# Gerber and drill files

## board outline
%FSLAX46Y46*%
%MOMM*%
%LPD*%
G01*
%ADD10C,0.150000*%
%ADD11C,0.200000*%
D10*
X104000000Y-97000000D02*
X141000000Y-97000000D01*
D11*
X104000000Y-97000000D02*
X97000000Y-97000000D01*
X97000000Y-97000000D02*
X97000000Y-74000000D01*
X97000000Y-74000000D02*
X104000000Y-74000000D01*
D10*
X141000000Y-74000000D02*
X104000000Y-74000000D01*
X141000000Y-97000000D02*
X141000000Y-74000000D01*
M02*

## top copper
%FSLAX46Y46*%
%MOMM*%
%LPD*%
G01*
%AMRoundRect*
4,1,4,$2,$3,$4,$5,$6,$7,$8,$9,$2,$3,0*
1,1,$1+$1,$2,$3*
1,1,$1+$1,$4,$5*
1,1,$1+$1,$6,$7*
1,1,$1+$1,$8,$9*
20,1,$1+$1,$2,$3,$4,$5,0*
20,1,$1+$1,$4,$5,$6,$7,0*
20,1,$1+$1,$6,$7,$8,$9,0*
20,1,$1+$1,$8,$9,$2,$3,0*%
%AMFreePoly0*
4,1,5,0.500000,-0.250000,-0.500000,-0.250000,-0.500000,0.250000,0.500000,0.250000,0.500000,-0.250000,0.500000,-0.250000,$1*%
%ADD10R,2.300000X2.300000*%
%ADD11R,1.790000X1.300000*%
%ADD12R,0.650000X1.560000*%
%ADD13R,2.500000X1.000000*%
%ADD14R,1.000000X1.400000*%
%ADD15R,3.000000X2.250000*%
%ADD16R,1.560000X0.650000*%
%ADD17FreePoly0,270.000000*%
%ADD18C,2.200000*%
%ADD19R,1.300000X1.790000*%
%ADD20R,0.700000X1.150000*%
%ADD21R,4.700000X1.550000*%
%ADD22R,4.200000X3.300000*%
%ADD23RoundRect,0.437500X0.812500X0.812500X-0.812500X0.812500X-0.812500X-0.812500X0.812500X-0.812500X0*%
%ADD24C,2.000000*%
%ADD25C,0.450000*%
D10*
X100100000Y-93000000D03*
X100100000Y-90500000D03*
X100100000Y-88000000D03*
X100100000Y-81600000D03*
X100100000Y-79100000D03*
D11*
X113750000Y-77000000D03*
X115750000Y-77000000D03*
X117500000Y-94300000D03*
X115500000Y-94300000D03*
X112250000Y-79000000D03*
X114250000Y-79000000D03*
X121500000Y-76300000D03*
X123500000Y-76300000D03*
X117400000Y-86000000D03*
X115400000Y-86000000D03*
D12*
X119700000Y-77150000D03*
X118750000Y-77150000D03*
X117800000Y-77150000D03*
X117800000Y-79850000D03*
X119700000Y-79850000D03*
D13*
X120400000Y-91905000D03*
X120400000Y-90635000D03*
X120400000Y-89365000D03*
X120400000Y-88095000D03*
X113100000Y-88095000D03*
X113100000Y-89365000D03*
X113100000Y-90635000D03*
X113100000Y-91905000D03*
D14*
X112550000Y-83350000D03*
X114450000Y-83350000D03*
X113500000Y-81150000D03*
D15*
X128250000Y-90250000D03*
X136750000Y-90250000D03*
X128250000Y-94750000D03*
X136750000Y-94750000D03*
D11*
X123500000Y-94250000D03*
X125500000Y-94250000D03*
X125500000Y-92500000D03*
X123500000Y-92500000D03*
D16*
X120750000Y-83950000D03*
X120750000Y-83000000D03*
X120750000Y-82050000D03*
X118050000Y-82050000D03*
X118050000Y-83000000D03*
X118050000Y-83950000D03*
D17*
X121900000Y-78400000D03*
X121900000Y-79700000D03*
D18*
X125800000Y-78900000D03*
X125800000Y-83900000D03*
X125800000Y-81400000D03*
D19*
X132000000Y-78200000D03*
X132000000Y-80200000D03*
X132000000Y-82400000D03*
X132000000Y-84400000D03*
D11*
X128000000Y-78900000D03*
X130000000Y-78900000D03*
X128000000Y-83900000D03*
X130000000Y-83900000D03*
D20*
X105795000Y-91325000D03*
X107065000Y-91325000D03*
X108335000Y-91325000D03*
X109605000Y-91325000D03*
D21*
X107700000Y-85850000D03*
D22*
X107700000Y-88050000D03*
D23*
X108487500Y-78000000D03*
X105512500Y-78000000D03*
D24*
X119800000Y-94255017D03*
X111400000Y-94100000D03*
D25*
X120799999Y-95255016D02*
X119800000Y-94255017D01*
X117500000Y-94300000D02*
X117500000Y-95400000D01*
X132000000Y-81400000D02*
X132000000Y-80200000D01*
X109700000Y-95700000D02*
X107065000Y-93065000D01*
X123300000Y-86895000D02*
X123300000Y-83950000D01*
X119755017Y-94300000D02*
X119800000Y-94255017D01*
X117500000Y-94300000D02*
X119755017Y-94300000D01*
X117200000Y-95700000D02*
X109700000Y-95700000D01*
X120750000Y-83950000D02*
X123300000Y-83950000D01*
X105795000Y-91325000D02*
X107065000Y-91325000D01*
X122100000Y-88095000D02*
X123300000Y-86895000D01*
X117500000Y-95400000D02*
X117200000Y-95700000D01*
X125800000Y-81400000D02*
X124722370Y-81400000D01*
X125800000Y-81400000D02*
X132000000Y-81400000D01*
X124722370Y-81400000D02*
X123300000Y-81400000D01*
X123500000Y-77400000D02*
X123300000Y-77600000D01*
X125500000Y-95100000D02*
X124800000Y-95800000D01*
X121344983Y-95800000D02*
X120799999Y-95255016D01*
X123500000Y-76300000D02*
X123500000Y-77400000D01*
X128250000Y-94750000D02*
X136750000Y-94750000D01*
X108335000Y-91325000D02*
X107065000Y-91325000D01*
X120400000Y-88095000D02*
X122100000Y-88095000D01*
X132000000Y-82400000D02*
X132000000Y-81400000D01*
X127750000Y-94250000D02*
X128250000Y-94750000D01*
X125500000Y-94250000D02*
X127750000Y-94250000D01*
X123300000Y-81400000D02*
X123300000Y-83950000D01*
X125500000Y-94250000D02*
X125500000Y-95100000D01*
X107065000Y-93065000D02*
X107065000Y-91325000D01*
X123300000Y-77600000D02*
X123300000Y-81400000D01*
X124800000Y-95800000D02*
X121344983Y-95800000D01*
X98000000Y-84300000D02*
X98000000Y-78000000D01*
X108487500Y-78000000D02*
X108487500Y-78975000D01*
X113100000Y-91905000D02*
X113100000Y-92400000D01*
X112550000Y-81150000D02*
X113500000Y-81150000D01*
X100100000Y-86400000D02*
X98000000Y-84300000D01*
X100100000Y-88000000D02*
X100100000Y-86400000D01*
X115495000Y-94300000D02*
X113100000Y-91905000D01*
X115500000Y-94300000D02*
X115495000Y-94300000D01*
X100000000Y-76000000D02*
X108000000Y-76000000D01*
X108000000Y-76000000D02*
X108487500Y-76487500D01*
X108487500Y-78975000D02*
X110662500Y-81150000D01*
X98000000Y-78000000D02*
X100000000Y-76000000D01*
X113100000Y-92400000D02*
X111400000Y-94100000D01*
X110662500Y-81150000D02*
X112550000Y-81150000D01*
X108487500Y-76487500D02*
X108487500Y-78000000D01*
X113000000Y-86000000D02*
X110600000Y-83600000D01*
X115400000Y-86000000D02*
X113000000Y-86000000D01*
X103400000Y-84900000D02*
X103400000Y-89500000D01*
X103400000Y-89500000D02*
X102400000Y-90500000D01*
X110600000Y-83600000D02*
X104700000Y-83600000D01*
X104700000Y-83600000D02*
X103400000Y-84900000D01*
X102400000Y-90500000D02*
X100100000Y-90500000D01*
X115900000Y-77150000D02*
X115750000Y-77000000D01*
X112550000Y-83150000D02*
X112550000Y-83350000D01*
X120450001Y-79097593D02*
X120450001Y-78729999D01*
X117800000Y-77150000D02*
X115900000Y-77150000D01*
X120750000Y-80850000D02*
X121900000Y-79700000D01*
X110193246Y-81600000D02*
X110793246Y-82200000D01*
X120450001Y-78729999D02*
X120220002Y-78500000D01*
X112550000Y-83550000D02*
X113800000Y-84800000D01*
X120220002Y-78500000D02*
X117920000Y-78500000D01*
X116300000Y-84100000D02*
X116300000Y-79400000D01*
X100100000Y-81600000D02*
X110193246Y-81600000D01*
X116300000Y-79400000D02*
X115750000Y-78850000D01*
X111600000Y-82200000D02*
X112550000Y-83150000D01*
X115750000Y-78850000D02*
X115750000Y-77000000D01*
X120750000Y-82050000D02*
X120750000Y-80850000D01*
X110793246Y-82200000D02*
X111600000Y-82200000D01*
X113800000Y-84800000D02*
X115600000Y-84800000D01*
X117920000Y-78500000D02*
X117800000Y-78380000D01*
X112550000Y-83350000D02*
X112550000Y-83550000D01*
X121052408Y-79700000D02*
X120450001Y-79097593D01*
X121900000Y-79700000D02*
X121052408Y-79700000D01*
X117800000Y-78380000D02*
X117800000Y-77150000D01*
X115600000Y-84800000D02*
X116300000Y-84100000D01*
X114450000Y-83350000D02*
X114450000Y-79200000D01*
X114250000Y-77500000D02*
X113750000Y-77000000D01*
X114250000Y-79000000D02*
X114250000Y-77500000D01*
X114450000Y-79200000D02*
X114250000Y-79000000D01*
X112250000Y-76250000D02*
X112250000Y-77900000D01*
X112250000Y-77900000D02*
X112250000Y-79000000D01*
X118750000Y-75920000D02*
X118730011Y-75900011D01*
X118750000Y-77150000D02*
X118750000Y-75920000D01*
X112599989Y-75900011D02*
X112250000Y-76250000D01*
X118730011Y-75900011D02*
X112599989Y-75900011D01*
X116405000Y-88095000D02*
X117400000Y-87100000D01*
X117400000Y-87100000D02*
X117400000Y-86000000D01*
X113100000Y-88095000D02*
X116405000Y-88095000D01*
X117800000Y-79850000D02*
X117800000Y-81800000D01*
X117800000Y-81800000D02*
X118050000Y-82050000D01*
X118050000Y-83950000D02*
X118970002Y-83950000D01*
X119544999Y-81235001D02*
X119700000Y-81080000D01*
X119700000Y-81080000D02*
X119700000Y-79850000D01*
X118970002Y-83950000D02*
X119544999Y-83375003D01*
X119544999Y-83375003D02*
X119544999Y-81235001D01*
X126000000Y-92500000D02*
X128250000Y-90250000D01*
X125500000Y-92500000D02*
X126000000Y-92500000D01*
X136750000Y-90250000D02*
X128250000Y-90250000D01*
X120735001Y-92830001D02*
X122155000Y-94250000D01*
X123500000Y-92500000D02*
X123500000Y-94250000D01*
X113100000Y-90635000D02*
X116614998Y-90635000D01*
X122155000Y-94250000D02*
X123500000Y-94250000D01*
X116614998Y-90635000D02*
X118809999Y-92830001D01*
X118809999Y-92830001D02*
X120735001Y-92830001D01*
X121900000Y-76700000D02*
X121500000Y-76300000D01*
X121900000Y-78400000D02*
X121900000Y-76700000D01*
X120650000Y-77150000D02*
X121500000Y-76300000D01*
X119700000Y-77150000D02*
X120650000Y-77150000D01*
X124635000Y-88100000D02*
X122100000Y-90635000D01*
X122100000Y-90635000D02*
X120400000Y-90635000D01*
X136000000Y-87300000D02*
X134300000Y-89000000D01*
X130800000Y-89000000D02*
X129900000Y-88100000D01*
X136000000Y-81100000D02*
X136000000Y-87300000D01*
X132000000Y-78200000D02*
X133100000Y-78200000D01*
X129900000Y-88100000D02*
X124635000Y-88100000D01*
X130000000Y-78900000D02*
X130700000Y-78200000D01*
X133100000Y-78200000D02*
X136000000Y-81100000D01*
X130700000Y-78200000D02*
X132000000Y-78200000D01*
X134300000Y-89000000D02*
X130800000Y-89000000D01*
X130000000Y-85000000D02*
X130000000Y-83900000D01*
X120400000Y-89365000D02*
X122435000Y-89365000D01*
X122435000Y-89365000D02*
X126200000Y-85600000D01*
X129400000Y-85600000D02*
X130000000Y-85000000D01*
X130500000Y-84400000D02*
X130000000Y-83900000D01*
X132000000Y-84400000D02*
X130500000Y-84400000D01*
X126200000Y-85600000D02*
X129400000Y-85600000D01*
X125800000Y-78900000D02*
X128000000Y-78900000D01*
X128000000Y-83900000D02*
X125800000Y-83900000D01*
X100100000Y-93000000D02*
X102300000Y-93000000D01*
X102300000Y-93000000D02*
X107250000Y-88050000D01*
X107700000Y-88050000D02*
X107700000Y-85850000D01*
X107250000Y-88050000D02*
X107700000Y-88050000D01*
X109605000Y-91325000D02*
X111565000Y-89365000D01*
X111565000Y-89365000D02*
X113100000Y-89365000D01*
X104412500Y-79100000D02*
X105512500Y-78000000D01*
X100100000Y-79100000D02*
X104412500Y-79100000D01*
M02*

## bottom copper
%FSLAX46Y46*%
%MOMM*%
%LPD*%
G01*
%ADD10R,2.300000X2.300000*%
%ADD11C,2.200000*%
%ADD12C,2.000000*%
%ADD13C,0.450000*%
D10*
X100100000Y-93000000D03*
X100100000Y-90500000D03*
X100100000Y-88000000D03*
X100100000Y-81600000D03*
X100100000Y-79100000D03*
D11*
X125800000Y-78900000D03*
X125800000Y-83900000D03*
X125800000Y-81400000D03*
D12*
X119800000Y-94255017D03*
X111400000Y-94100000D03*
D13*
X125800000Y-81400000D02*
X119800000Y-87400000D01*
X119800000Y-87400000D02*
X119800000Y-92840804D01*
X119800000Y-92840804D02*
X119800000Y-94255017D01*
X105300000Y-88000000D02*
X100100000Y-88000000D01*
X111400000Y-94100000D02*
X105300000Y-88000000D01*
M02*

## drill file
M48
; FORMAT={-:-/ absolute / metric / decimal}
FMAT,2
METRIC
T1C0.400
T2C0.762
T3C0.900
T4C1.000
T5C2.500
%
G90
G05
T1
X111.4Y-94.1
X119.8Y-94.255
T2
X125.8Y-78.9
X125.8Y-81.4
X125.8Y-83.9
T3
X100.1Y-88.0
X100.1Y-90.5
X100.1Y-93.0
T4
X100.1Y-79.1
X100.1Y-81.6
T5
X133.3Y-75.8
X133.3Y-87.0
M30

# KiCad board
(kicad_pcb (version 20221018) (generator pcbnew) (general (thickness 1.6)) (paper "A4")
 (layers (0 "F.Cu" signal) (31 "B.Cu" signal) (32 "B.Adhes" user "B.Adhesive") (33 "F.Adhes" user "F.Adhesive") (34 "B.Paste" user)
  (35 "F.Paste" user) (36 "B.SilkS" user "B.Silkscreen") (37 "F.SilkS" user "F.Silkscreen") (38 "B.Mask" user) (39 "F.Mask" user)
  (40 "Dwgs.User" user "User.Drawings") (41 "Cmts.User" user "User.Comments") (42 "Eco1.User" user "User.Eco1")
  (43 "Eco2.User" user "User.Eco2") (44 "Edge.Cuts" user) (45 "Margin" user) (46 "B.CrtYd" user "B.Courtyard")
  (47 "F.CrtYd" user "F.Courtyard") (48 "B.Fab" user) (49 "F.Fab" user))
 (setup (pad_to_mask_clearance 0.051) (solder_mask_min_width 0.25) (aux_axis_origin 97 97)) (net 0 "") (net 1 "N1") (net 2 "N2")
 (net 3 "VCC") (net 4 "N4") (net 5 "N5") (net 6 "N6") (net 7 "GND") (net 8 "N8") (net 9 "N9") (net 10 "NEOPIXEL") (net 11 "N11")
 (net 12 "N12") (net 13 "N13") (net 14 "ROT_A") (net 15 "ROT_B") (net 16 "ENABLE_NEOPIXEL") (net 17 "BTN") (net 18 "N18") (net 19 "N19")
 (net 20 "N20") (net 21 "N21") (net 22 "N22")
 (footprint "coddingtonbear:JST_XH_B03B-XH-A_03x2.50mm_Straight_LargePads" (layer "F.Cu") (at 100.1 93 90)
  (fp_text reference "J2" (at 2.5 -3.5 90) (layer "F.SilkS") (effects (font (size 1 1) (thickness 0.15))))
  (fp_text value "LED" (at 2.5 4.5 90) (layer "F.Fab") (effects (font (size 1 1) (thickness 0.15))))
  (pad "1" thru_hole rect (at 0 0 90) (size 2.3 2.3) (drill 0.9) (layers "*.Cu" "*.Mask") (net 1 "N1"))
  (pad "2" thru_hole rect (at 2.5 0 90) (size 2.3 2.3) (drill 0.9) (layers "*.Cu" "*.Mask") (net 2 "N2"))
  (pad "3" thru_hole rect (at 5 0 90) (size 2.3 2.3) (drill 0.9) (layers "*.Cu" "*.Mask") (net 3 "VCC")))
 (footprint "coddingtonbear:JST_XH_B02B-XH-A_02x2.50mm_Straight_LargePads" (layer "F.Cu") (at 100.1 81.6 90)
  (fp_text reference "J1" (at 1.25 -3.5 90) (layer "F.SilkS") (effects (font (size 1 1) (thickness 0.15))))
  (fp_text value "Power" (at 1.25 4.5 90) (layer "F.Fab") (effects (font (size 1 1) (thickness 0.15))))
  (pad "1" thru_hole rect (at 0 0 90) (size 2.3 2.3) (drill 1) (layers "*.Cu" "*.Mask") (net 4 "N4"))
  (pad "2" thru_hole rect (at 2.5 0 90) (size 2.3 2.3) (drill 1) (layers "*.Cu" "*.Mask") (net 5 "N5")))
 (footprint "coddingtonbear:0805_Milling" (layer "F.Cu") (at 114.75 77)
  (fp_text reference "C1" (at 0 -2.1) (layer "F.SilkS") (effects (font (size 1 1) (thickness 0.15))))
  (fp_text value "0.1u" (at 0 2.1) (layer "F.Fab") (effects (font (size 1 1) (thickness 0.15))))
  (pad "1" smd rect (at -1 0) (size 1.79 1.3) (layers "F.Cu" "F.Paste" "F.Mask") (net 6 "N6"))
  (pad "2" smd rect (at 1 0) (size 1.79 1.3) (layers "F.Cu" "F.Paste" "F.Mask") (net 4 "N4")))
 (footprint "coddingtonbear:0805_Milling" (layer "F.Cu") (at 116.5 94.3 180)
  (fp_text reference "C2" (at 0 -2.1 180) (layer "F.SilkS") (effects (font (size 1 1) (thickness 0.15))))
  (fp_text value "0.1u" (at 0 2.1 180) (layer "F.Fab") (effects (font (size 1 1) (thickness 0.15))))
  (pad "1" smd rect (at -1 0 180) (size 1.79 1.3) (layers "F.Cu" "F.Paste" "F.Mask") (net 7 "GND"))
  (pad "2" smd rect (at 1 0 180) (size 1.79 1.3) (layers "F.Cu" "F.Paste" "F.Mask") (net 3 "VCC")))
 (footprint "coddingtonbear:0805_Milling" (layer "F.Cu") (at 113.25 79)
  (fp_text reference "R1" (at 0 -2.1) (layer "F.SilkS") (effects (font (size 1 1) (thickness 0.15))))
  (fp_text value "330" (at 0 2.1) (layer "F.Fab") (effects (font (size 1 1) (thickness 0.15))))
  (pad "1" smd rect (at -1 0) (size 1.79 1.3) (layers "F.Cu" "F.Paste" "F.Mask") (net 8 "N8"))
  (pad "2" smd rect (at 1 0) (size 1.79 1.3) (layers "F.Cu" "F.Paste" "F.Mask") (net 6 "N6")))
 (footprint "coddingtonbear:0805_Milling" (layer "F.Cu") (at 122.5 76.3)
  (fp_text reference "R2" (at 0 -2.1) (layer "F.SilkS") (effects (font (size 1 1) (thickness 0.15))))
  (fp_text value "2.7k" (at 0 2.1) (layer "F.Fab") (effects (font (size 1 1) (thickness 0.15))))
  (pad "1" smd rect (at -1 0) (size 1.79 1.3) (layers "F.Cu" "F.Paste" "F.Mask") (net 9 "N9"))
  (pad "2" smd rect (at 1 0) (size 1.79 1.3) (layers "F.Cu" "F.Paste" "F.Mask") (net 7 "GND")))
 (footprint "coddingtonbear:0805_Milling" (layer "F.Cu") (at 116.4 86 180)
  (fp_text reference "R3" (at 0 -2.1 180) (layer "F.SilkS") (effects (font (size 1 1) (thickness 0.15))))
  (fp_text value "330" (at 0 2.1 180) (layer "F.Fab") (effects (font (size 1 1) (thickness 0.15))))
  (pad "1" smd rect (at -1 0 180) (size 1.79 1.3) (layers "F.Cu" "F.Paste" "F.Mask") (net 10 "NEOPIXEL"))
  (pad "2" smd rect (at 1 0 180) (size 1.79 1.3) (layers "F.Cu" "F.Paste" "F.Mask") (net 2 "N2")))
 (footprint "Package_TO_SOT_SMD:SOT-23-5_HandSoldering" (layer "F.Cu") (at 118.75 78.5 -90)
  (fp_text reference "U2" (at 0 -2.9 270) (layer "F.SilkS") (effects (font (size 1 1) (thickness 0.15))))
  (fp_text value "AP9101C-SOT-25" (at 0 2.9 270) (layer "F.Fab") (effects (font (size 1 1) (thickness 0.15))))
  (pad "1" smd rect (at -1.35 -0.95 270) (size 1.56 0.65) (layers "F.Cu" "F.Paste" "F.Mask") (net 9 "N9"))
  (pad "2" smd rect (at -1.35 0 270) (size 1.56 0.65) (layers "F.Cu" "F.Paste" "F.Mask") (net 8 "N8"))
  (pad "3" smd rect (at -1.35 0.95 270) (size 1.56 0.65) (layers "F.Cu" "F.Paste" "F.Mask") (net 4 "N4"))
  (pad "4" smd rect (at 1.35 0.95 270) (size 1.56 0.65) (layers "F.Cu" "F.Paste" "F.Mask") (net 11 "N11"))
  (pad "5" smd rect (at 1.35 -0.95 270) (size 1.56 0.65) (layers "F.Cu" "F.Paste" "F.Mask") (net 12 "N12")))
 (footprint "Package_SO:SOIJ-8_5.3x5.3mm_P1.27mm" (layer "F.Cu") (at 116.75 90 180)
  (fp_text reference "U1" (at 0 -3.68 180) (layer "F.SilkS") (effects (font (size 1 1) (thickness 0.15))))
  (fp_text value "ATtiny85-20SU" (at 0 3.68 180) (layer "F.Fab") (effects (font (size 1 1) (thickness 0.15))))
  (pad "1" smd rect (at -3.65 -1.905 180) (size 2.5 1) (layers "F.Cu" "F.Paste" "F.Mask") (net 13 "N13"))
  (pad "2" smd rect (at -3.65 -0.635 180) (size 2.5 1) (layers "F.Cu" "F.Paste" "F.Mask") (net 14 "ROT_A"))
  (pad "3" smd rect (at -3.65 0.635 180) (size 2.5 1) (layers "F.Cu" "F.Paste" "F.Mask") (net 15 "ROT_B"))
  (pad "4" smd rect (at -3.65 1.905 180) (size 2.5 1) (layers "F.Cu" "F.Paste" "F.Mask") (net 7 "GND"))
  (pad "5" smd rect (at 3.65 1.905 180) (size 2.5 1) (layers "F.Cu" "F.Paste" "F.Mask") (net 10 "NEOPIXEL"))
  (pad "6" smd rect (at 3.65 0.635 180) (size 2.5 1) (layers "F.Cu" "F.Paste" "F.Mask") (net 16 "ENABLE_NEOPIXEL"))
  (pad "7" smd rect (at 3.65 -0.635 180) (size 2.5 1) (layers "F.Cu" "F.Paste" "F.Mask") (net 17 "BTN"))
  (pad "8" smd rect (at 3.65 -1.905 180) (size 2.5 1) (layers "F.Cu" "F.Paste" "F.Mask") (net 3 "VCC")))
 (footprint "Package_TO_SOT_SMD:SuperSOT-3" (layer "F.Cu") (at 113.5 82.25 90)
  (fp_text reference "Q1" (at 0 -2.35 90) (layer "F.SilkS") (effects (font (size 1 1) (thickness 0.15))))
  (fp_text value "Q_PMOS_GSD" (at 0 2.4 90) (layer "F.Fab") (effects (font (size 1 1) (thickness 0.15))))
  (pad "1" smd rect (at -1.1 -0.95 90) (size 1.4 1) (layers "F.Cu" "F.Paste" "F.Mask") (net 4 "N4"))
  (pad "2" smd rect (at -1.1 0.95 90) (size 1.4 1) (layers "F.Cu" "F.Paste" "F.Mask") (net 6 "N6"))
  (pad "3" smd rect (at 1.1 0 90) (size 1.4 1) (layers "F.Cu" "F.Paste" "F.Mask") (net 3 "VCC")))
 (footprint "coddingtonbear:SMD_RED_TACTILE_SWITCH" (layer "F.Cu") (at 132.5 92.5)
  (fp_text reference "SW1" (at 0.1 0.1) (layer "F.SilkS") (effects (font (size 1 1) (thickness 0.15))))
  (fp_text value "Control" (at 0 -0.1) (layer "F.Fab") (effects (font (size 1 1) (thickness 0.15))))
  (pad "1" smd rect (at -4.25 -2.25) (size 3 2.25) (layers "F.Cu" "F.Paste" "F.Mask") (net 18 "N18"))
  (pad "1" smd rect (at 4.25 -2.25) (size 3 2.25) (layers "F.Cu" "F.Paste" "F.Mask") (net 18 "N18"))
  (pad "2" smd rect (at -4.25 2.25) (size 3 2.25) (layers "F.Cu" "F.Paste" "F.Mask") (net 7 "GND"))
  (pad "2" smd rect (at 4.25 2.25) (size 3 2.25) (layers "F.Cu" "F.Paste" "F.Mask") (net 7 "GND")))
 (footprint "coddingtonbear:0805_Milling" (layer "F.Cu") (at 124.5 94.25)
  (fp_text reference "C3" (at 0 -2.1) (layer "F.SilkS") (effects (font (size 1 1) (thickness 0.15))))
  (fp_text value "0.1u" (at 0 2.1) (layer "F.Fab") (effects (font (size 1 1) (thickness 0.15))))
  (pad "1" smd rect (at -1 0) (size 1.79 1.3) (layers "F.Cu" "F.Paste" "F.Mask") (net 17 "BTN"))
  (pad "2" smd rect (at 1 0) (size 1.79 1.3) (layers "F.Cu" "F.Paste" "F.Mask") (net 7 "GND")))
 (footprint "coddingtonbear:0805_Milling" (layer "F.Cu") (at 124.5 92.5 180)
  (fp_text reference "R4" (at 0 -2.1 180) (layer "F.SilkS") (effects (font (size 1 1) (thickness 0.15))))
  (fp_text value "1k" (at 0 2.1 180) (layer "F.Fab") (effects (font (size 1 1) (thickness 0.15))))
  (pad "1" smd rect (at -1 0 180) (size 1.79 1.3) (layers "F.Cu" "F.Paste" "F.Mask") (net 18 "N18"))
  (pad "2" smd rect (at 1 0 180) (size 1.79 1.3) (layers "F.Cu" "F.Paste" "F.Mask") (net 17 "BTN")))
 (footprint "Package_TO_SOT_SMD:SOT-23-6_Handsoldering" (layer "F.Cu") (at 119.4 83 180)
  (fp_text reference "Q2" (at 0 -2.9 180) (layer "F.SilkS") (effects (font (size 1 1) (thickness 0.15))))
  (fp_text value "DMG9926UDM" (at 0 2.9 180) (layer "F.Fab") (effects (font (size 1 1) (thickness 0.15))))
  (pad "1" smd rect (at -1.35 -0.95 180) (size 1.56 0.65) (layers "F.Cu" "F.Paste" "F.Mask") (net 7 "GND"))
  (pad "2" smd rect (at -1.35 0 180) (size 1.56 0.65) (layers "F.Cu" "F.Paste" "F.Mask") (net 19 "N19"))
  (pad "3" smd rect (at -1.35 0.95 180) (size 1.56 0.65) (layers "F.Cu" "F.Paste" "F.Mask") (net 4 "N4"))
  (pad "4" smd rect (at 1.35 0.95 180) (size 1.56 0.65) (layers "F.Cu" "F.Paste" "F.Mask") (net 11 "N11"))
  (pad "5" smd rect (at 1.35 0 180) (size 1.56 0.65) (layers "F.Cu" "F.Paste" "F.Mask") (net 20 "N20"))
  (pad "6" smd rect (at 1.35 -0.95 180) (size 1.56 0.65) (layers "F.Cu" "F.Paste" "F.Mask") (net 12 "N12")))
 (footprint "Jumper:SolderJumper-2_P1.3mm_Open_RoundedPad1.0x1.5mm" (layer "F.Cu") (at 121.9 79.05 -90)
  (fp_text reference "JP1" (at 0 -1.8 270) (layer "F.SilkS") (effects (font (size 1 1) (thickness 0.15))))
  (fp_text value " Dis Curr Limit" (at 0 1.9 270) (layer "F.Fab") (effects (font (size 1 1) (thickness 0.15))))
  (pad "1" smd custom (at -0.65 0 270) (size 1 0.5) (layers "F.Cu" "F.Mask") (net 9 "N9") (zone_connect 0) (thermal_bridge_angle 45)
   (options (clearance outline) (anchor rect)) (primitives))
  (pad "2" smd custom (at 0.65 0 270) (size 1 0.5) (layers "F.Cu" "F.Mask") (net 4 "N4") (zone_connect 0) (thermal_bridge_angle 45)
   (options (clearance outline) (anchor rect)) (primitives)))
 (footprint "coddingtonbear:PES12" (layer "F.Cu") (at 133.3 81.4 -90)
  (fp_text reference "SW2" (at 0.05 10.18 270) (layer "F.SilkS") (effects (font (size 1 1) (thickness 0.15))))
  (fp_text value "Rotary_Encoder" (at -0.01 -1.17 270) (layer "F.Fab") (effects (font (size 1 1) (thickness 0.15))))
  (pad "" np_thru_hole circle (at -5.6 0 270) (size 2.5 2.5) (drill 2.5) (layers "*.Cu" "*.Mask"))
  (pad "" np_thru_hole circle (at 5.6 0 270) (size 2.5 2.5) (drill 2.5) (layers "*.Cu" "*.Mask"))
  (pad "A" thru_hole circle (at -2.5 7.5 270) (size 2.2 2.2) (drill 0.762) (layers "*.Cu" "*.Mask") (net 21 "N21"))
  (pad "B" thru_hole circle (at 2.5 7.5 270) (size 2.2 2.2) (drill 0.762) (layers "*.Cu" "*.Mask") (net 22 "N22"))
  (pad "C" thru_hole circle (at 0 7.5 270) (size 2.2 2.2) (drill 0.762) (layers "*.Cu" "*.Mask") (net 7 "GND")))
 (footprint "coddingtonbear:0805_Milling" (layer "F.Cu") (at 132 79.2 -90)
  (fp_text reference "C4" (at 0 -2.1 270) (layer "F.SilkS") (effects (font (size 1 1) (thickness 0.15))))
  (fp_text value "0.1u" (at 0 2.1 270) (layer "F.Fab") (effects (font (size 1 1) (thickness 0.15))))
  (pad "1" smd rect (at -1 0 270) (size 1.79 1.3) (layers "F.Cu" "F.Paste" "F.Mask") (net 14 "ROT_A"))
  (pad "2" smd rect (at 1 0 270) (size 1.79 1.3) (layers "F.Cu" "F.Paste" "F.Mask") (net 7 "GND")))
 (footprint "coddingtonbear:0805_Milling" (layer "F.Cu") (at 132 83.4 -90)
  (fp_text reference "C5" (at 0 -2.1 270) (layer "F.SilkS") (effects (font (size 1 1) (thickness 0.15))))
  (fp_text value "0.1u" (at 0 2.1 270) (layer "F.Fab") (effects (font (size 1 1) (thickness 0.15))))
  (pad "1" smd rect (at -1 0 270) (size 1.79 1.3) (layers "F.Cu" "F.Paste" "F.Mask") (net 7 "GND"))
  (pad "2" smd rect (at 1 0 270) (size 1.79 1.3) (layers "F.Cu" "F.Paste" "F.Mask") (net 15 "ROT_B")))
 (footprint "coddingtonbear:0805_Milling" (layer "F.Cu") (at 129 78.9)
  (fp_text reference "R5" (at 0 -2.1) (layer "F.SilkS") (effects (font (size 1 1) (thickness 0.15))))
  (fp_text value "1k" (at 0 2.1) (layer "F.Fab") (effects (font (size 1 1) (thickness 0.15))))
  (pad "1" smd rect (at -1 0) (size 1.79 1.3) (layers "F.Cu" "F.Paste" "F.Mask") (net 21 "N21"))
  (pad "2" smd rect (at 1 0) (size 1.79 1.3) (layers "F.Cu" "F.Paste" "F.Mask") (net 14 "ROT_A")))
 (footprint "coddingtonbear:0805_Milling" (layer "F.Cu") (at 129 83.9)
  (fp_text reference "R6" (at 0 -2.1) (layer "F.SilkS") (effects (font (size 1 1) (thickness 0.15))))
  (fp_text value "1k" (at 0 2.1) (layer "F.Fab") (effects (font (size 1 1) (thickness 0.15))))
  (pad "1" smd rect (at -1 0) (size 1.79 1.3) (layers "F.Cu" "F.Paste" "F.Mask") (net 22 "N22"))
  (pad "2" smd rect (at 1 0) (size 1.79 1.3) (layers "F.Cu" "F.Paste" "F.Mask") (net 15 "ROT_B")))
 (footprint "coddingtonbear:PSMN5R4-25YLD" (layer "F.Cu") (at 107.7 88.5)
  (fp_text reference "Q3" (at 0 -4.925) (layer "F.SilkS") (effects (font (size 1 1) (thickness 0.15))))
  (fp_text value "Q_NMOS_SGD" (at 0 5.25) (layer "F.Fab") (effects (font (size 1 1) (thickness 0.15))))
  (pad "" smd rect (at -1.875 -2.9) (size 0.6 0.9) (layers "F.Paste"))
  (pad "" smd rect (at -1.15 -1.05 90) (size 0.6 0.9) (layers "F.Paste"))
  (pad "" smd rect (at -1.15 -0.2 90) (size 0.6 0.9) (layers "F.Paste"))
  (pad "" smd rect (at -1.15 0.65 90) (size 0.6 0.9) (layers "F.Paste"))
  (pad "" smd rect (at -0.6 -2.9) (size 0.6 0.9) (layers "F.Paste"))
  (pad "" smd rect (at 0 -1.05 90) (size 0.6 0.9) (layers "F.Paste"))
  (pad "" smd rect (at 0 -0.2 90) (size 0.6 0.9) (layers "F.Paste"))
  (pad "" smd rect (at 0 0.65 90) (size 0.6 0.9) (layers "F.Paste"))
  (pad "" smd rect (at 0.6 -2.9) (size 0.6 0.9) (layers "F.Paste"))
  (pad "" smd rect (at 1.15 -1.05 90) (size 0.6 0.9) (layers "F.Paste"))
  (pad "" smd rect (at 1.15 -0.2 90) (size 0.6 0.9) (layers "F.Paste"))
  (pad "" smd rect (at 1.15 0.65 90) (size 0.6 0.9) (layers "F.Paste"))
  (pad "" smd rect (at 1.875 -2.9) (size 0.6 0.9) (layers "F.Paste"))
  (pad "1" smd rect (at -1.905 2.825) (size 0.7 1.15) (layers "F.Cu" "F.Paste" "F.Mask") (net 7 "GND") (solder_mask_margin 0.075)
   (solder_paste_margin -0.05))
  (pad "1" smd rect (at -0.635 2.825) (size 0.7 1.15) (layers "F.Cu" "F.Paste" "F.Mask") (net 7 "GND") (solder_mask_margin 0.075)
   (solder_paste_margin -0.05))
  (pad "1" smd rect (at 0.635 2.825) (size 0.7 1.15) (layers "F.Cu" "F.Paste" "F.Mask") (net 7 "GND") (solder_mask_margin 0.075)
   (solder_paste_margin -0.05))
  (pad "2" smd rect (at 1.905 2.825) (size 0.7 1.15) (layers "F.Cu" "F.Paste" "F.Mask") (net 16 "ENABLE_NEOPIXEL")
   (solder_mask_margin 0.075) (solder_paste_margin -0.05))
  (pad "3" smd rect (at 0 -2.65) (size 4.7 1.55) (layers "F.Cu" "F.Mask") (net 1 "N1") (solder_mask_margin 0.075))
  (pad "3" smd rect (at 0 -0.45) (size 4.2 3.3) (layers "F.Cu" "F.Mask") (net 1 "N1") (solder_mask_margin 0.075)))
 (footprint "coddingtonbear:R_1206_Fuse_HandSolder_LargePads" (layer "F.Cu") (at 107 78 180)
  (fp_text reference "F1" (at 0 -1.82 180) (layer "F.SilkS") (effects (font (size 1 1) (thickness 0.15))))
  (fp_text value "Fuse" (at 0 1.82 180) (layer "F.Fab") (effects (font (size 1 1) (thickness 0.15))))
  (pad "1" smd roundrect (at -1.4875 0 180) (size 2.5 2.5) (layers "F.Cu" "F.Paste" "F.Mask") (roundrect_rratio 0.175) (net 3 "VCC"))
  (pad "2" smd roundrect (at 1.4875 0 180) (size 2.5 2.5) (layers "F.Cu" "F.Paste" "F.Mask") (roundrect_rratio 0.175) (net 5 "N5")))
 (gr_line (start 104 97) (end 141 97) (stroke (width 0.15) (type solid)) (layer "Edge.Cuts"))
 (gr_line (start 104 97) (end 97 97) (stroke (width 0.2) (type solid)) (layer "Edge.Cuts"))
 (gr_line (start 97 97) (end 97 74) (stroke (width 0.2) (type solid)) (layer "Edge.Cuts"))
 (gr_line (start 97 74) (end 104 74) (stroke (width 0.2) (type solid)) (layer "Edge.Cuts"))
 (gr_line (start 141 74) (end 104 74) (stroke (width 0.15) (type solid)) (layer "Edge.Cuts"))
 (gr_line (start 141 97) (end 141 74) (stroke (width 0.15) (type solid)) (layer "Edge.Cuts"))
 (segment (start 120.799999 95.255016) (end 119.8 94.255017) (width 0.45) (layer "F.Cu") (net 7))
 (segment (start 117.5 94.3) (end 117.5 95.4) (width 0.45) (layer "F.Cu") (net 7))
 (segment (start 132 81.4) (end 132 80.2) (width 0.45) (layer "F.Cu") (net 7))
 (segment (start 109.7 95.7) (end 107.065 93.065) (width 0.45) (layer "F.Cu") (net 7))
 (segment (start 123.3 86.895) (end 123.3 83.95) (width 0.45) (layer "F.Cu") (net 7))
 (segment (start 119.755017 94.3) (end 119.8 94.255017) (width 0.45) (layer "F.Cu") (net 7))
 (segment (start 117.5 94.3) (end 119.755017 94.3) (width 0.45) (layer "F.Cu") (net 7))
 (segment (start 117.2 95.7) (end 109.7 95.7) (width 0.45) (layer "F.Cu") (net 7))
 (segment (start 120.75 83.95) (end 123.3 83.95) (width 0.45) (layer "F.Cu") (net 7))
 (segment (start 105.795 91.325) (end 107.065 91.325) (width 0.45) (layer "F.Cu") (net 7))
 (segment (start 122.1 88.095) (end 123.3 86.895) (width 0.45) (layer "F.Cu") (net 7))
 (segment (start 117.5 95.4) (end 117.2 95.7) (width 0.45) (layer "F.Cu") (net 7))
 (segment (start 125.8 81.4) (end 124.72237 81.4) (width 0.45) (layer "F.Cu") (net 7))
 (segment (start 125.8 81.4) (end 132 81.4) (width 0.45) (layer "F.Cu") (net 7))
 (segment (start 124.72237 81.4) (end 123.3 81.4) (width 0.45) (layer "F.Cu") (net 7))
 (segment (start 123.5 77.4) (end 123.3 77.6) (width 0.45) (layer "F.Cu") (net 7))
 (segment (start 125.5 95.1) (end 124.8 95.8) (width 0.45) (layer "F.Cu") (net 7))
 (segment (start 121.344983 95.8) (end 120.799999 95.255016) (width 0.45) (layer "F.Cu") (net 7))
 (segment (start 123.5 76.3) (end 123.5 77.4) (width 0.45) (layer "F.Cu") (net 7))
 (segment (start 128.25 94.75) (end 136.75 94.75) (width 0.45) (layer "F.Cu") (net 7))
 (segment (start 108.335 91.325) (end 107.065 91.325) (width 0.45) (layer "F.Cu") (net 7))
 (segment (start 120.4 88.095) (end 122.1 88.095) (width 0.45) (layer "F.Cu") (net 7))
 (segment (start 132 82.4) (end 132 81.4) (width 0.45) (layer "F.Cu") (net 7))
 (segment (start 127.75 94.25) (end 128.25 94.75) (width 0.45) (layer "F.Cu") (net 7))
 (segment (start 125.5 94.25) (end 127.75 94.25) (width 0.45) (layer "F.Cu") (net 7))
 (segment (start 123.3 81.4) (end 123.3 83.95) (width 0.45) (layer "F.Cu") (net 7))
 (segment (start 125.5 94.25) (end 125.5 95.1) (width 0.45) (layer "F.Cu") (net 7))
 (segment (start 107.065 93.065) (end 107.065 91.325) (width 0.45) (layer "F.Cu") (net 7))
 (segment (start 123.3 77.6) (end 123.3 81.4) (width 0.45) (layer "F.Cu") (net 7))
 (segment (start 124.8 95.8) (end 121.344983 95.8) (width 0.45) (layer "F.Cu") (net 7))
 (via (at 119.8 94.255017) (size 2) (drill 0.4) (layers "F.Cu" "B.Cu") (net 7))
 (segment (start 125.8 81.4) (end 119.8 87.4) (width 0.45) (layer "B.Cu") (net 7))
 (segment (start 119.8 87.4) (end 119.8 92.840804) (width 0.45) (layer "B.Cu") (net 7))
 (segment (start 119.8 92.840804) (end 119.8 94.255017) (width 0.45) (layer "B.Cu") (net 7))
 (segment (start 98 84.3) (end 98 78) (width 0.45) (layer "F.Cu") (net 3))
 (segment (start 108.4875 78) (end 108.4875 78.975) (width 0.45) (layer "F.Cu") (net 3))
 (segment (start 113.1 91.905) (end 113.1 92.4) (width 0.45) (layer "F.Cu") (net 3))
 (segment (start 112.55 81.15) (end 113.5 81.15) (width 0.45) (layer "F.Cu") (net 3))
 (segment (start 100.1 86.4) (end 98 84.3) (width 0.45) (layer "F.Cu") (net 3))
 (segment (start 100.1 88) (end 100.1 86.4) (width 0.45) (layer "F.Cu") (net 3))
 (segment (start 115.495 94.3) (end 113.1 91.905) (width 0.45) (layer "F.Cu") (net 3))
 (segment (start 115.5 94.3) (end 115.495 94.3) (width 0.45) (layer "F.Cu") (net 3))
 (segment (start 100 76) (end 108 76) (width 0.45) (layer "F.Cu") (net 3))
 (segment (start 108 76) (end 108.4875 76.4875) (width 0.45) (layer "F.Cu") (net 3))
 (segment (start 108.4875 78.975) (end 110.6625 81.15) (width 0.45) (layer "F.Cu") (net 3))
 (segment (start 98 78) (end 100 76) (width 0.45) (layer "F.Cu") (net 3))
 (segment (start 113.1 92.4) (end 111.4 94.1) (width 0.45) (layer "F.Cu") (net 3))
 (segment (start 110.6625 81.15) (end 112.55 81.15) (width 0.45) (layer "F.Cu") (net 3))
 (segment (start 108.4875 76.4875) (end 108.4875 78) (width 0.45) (layer "F.Cu") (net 3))
 (via (at 111.4 94.1) (size 2) (drill 0.4) (layers "F.Cu" "B.Cu") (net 3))
 (segment (start 105.3 88) (end 100.1 88) (width 0.45) (layer "B.Cu") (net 3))
 (segment (start 111.4 94.1) (end 105.3 88) (width 0.45) (layer "B.Cu") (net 3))
 (segment (start 113 86) (end 110.6 83.6) (width 0.45) (layer "F.Cu") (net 2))
 (segment (start 115.4 86) (end 113 86) (width 0.45) (layer "F.Cu") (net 2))
 (segment (start 103.4 84.9) (end 103.4 89.5) (width 0.45) (layer "F.Cu") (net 2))
 (segment (start 103.4 89.5) (end 102.4 90.5) (width 0.45) (layer "F.Cu") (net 2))
 (segment (start 110.6 83.6) (end 104.7 83.6) (width 0.45) (layer "F.Cu") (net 2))
 (segment (start 104.7 83.6) (end 103.4 84.9) (width 0.45) (layer "F.Cu") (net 2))
 (segment (start 102.4 90.5) (end 100.1 90.5) (width 0.45) (layer "F.Cu") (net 2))
 (segment (start 115.9 77.15) (end 115.75 77) (width 0.45) (layer "F.Cu") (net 4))
 (segment (start 112.55 83.15) (end 112.55 83.35) (width 0.45) (layer "F.Cu") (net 4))
 (segment (start 120.450001 79.097593) (end 120.450001 78.729999) (width 0.45) (layer "F.Cu") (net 4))
 (segment (start 117.8 77.15) (end 115.9 77.15) (width 0.45) (layer "F.Cu") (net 4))
 (segment (start 120.75 80.85) (end 121.9 79.7) (width 0.45) (layer "F.Cu") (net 4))
 (segment (start 110.193246 81.6) (end 110.793246 82.2) (width 0.45) (layer "F.Cu") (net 4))
 (segment (start 120.450001 78.729999) (end 120.220002 78.5) (width 0.45) (layer "F.Cu") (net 4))
 (segment (start 112.55 83.55) (end 113.8 84.8) (width 0.45) (layer "F.Cu") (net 4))
 (segment (start 120.220002 78.5) (end 117.92 78.5) (width 0.45) (layer "F.Cu") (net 4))
 (segment (start 116.3 84.1) (end 116.3 79.4) (width 0.45) (layer "F.Cu") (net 4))
 (segment (start 100.1 81.6) (end 110.193246 81.6) (width 0.45) (layer "F.Cu") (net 4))
 (segment (start 116.3 79.4) (end 115.75 78.85) (width 0.45) (layer "F.Cu") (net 4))
 (segment (start 111.6 82.2) (end 112.55 83.15) (width 0.45) (layer "F.Cu") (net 4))
 (segment (start 115.75 78.85) (end 115.75 77) (width 0.45) (layer "F.Cu") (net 4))
 (segment (start 120.75 82.05) (end 120.75 80.85) (width 0.45) (layer "F.Cu") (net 4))
 (segment (start 110.793246 82.2) (end 111.6 82.2) (width 0.45) (layer "F.Cu") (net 4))
 (segment (start 113.8 84.8) (end 115.6 84.8) (width 0.45) (layer "F.Cu") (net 4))
 (segment (start 117.92 78.5) (end 117.8 78.38) (width 0.45) (layer "F.Cu") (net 4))
 (segment (start 112.55 83.35) (end 112.55 83.55) (width 0.45) (layer "F.Cu") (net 4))
 (segment (start 121.052408 79.7) (end 120.450001 79.097593) (width 0.45) (layer "F.Cu") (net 4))
 (segment (start 121.9 79.7) (end 121.052408 79.7) (width 0.45) (layer "F.Cu") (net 4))
 (segment (start 117.8 78.38) (end 117.8 77.15) (width 0.45) (layer "F.Cu") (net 4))
 (segment (start 115.6 84.8) (end 116.3 84.1) (width 0.45) (layer "F.Cu") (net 4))
 (segment (start 114.45 83.35) (end 114.45 79.2) (width 0.45) (layer "F.Cu") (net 6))
 (segment (start 114.25 77.5) (end 113.75 77) (width 0.45) (layer "F.Cu") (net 6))
 (segment (start 114.25 79) (end 114.25 77.5) (width 0.45) (layer "F.Cu") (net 6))
 (segment (start 114.45 79.2) (end 114.25 79) (width 0.45) (layer "F.Cu") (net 6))
 (segment (start 112.25 76.25) (end 112.25 77.9) (width 0.45) (layer "F.Cu") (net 8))
 (segment (start 112.25 77.9) (end 112.25 79) (width 0.45) (layer "F.Cu") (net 8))
 (segment (start 118.75 75.92) (end 118.730011 75.900011) (width 0.45) (layer "F.Cu") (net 8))
 (segment (start 118.75 77.15) (end 118.75 75.92) (width 0.45) (layer "F.Cu") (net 8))
 (segment (start 112.599989 75.900011) (end 112.25 76.25) (width 0.45) (layer "F.Cu") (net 8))
 (segment (start 118.730011 75.900011) (end 112.599989 75.900011) (width 0.45) (layer "F.Cu") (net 8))
 (segment (start 116.405 88.095) (end 117.4 87.1) (width 0.45) (layer "F.Cu") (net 10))
 (segment (start 117.4 87.1) (end 117.4 86) (width 0.45) (layer "F.Cu") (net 10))
 (segment (start 113.1 88.095) (end 116.405 88.095) (width 0.45) (layer "F.Cu") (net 10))
 (segment (start 117.8 79.85) (end 117.8 81.8) (width 0.45) (layer "F.Cu") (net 11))
 (segment (start 117.8 81.8) (end 118.05 82.05) (width 0.45) (layer "F.Cu") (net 11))
 (segment (start 118.05 83.95) (end 118.970002 83.95) (width 0.45) (layer "F.Cu") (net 12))
 (segment (start 119.544999 81.235001) (end 119.7 81.08) (width 0.45) (layer "F.Cu") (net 12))
 (segment (start 119.7 81.08) (end 119.7 79.85) (width 0.45) (layer "F.Cu") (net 12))
 (segment (start 118.970002 83.95) (end 119.544999 83.375003) (width 0.45) (layer "F.Cu") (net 12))
 (segment (start 119.544999 83.375003) (end 119.544999 81.235001) (width 0.45) (layer "F.Cu") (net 12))
 (segment (start 126 92.5) (end 128.25 90.25) (width 0.45) (layer "F.Cu") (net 18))
 (segment (start 125.5 92.5) (end 126 92.5) (width 0.45) (layer "F.Cu") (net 18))
 (segment (start 136.75 90.25) (end 128.25 90.25) (width 0.45) (layer "F.Cu") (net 18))
 (segment (start 120.735001 92.830001) (end 122.155 94.25) (width 0.45) (layer "F.Cu") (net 17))
 (segment (start 123.5 92.5) (end 123.5 94.25) (width 0.45) (layer "F.Cu") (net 17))
 (segment (start 113.1 90.635) (end 116.614998 90.635) (width 0.45) (layer "F.Cu") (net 17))
 (segment (start 122.155 94.25) (end 123.5 94.25) (width 0.45) (layer "F.Cu") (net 17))
 (segment (start 116.614998 90.635) (end 118.809999 92.830001) (width 0.45) (layer "F.Cu") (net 17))
 (segment (start 118.809999 92.830001) (end 120.735001 92.830001) (width 0.45) (layer "F.Cu") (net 17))
 (segment (start 121.9 76.7) (end 121.5 76.3) (width 0.45) (layer "F.Cu") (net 9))
 (segment (start 121.9 78.4) (end 121.9 76.7) (width 0.45) (layer "F.Cu") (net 9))
 (segment (start 120.65 77.15) (end 121.5 76.3) (width 0.45) (layer "F.Cu") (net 9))
 (segment (start 119.7 77.15) (end 120.65 77.15) (width 0.45) (layer "F.Cu") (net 9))
 (segment (start 124.635 88.1) (end 122.1 90.635) (width 0.45) (layer "F.Cu") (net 14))
 (segment (start 122.1 90.635) (end 120.4 90.635) (width 0.45) (layer "F.Cu") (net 14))
 (segment (start 136 87.3) (end 134.3 89) (width 0.45) (layer "F.Cu") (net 14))
 (segment (start 130.8 89) (end 129.9 88.1) (width 0.45) (layer "F.Cu") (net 14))
 (segment (start 136 81.1) (end 136 87.3) (width 0.45) (layer "F.Cu") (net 14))
 (segment (start 132 78.2) (end 133.1 78.2) (width 0.45) (layer "F.Cu") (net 14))
 (segment (start 129.9 88.1) (end 124.635 88.1) (width 0.45) (layer "F.Cu") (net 14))
 (segment (start 130 78.9) (end 130.7 78.2) (width 0.45) (layer "F.Cu") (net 14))
 (segment (start 133.1 78.2) (end 136 81.1) (width 0.45) (layer "F.Cu") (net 14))
 (segment (start 130.7 78.2) (end 132 78.2) (width 0.45) (layer "F.Cu") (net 14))
 (segment (start 134.3 89) (end 130.8 89) (width 0.45) (layer "F.Cu") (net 14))
 (segment (start 130 85) (end 130 83.9) (width 0.45) (layer "F.Cu") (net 15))
 (segment (start 120.4 89.365) (end 122.435 89.365) (width 0.45) (layer "F.Cu") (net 15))
 (segment (start 122.435 89.365) (end 126.2 85.6) (width 0.45) (layer "F.Cu") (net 15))
 (segment (start 129.4 85.6) (end 130 85) (width 0.45) (layer "F.Cu") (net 15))
 (segment (start 130.5 84.4) (end 130 83.9) (width 0.45) (layer "F.Cu") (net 15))
 (segment (start 132 84.4) (end 130.5 84.4) (width 0.45) (layer "F.Cu") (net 15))
 (segment (start 126.2 85.6) (end 129.4 85.6) (width 0.45) (layer "F.Cu") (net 15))
 (segment (start 125.8 78.9) (end 128 78.9) (width 0.45) (layer "F.Cu") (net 21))
 (segment (start 128 83.9) (end 125.8 83.9) (width 0.45) (layer "F.Cu") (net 22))
 (segment (start 100.1 93) (end 102.3 93) (width 0.45) (layer "F.Cu") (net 1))
 (segment (start 102.3 93) (end 107.25 88.05) (width 0.45) (layer "F.Cu") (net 1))
 (segment (start 107.7 88.05) (end 107.7 85.85) (width 0.45) (layer "F.Cu") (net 1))
 (segment (start 107.25 88.05) (end 107.7 88.05) (width 0.45) (layer "F.Cu") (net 1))
 (segment (start 109.605 91.325) (end 111.565 89.365) (width 0.45) (layer "F.Cu") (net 16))
 (segment (start 111.565 89.365) (end 113.1 89.365) (width 0.45) (layer "F.Cu") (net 16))
 (segment (start 104.4125 79.1) (end 105.5125 78) (width 0.45) (layer "F.Cu") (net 5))
 (segment (start 100.1 79.1) (end 104.4125 79.1) (width 0.45) (layer "F.Cu") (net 5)))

